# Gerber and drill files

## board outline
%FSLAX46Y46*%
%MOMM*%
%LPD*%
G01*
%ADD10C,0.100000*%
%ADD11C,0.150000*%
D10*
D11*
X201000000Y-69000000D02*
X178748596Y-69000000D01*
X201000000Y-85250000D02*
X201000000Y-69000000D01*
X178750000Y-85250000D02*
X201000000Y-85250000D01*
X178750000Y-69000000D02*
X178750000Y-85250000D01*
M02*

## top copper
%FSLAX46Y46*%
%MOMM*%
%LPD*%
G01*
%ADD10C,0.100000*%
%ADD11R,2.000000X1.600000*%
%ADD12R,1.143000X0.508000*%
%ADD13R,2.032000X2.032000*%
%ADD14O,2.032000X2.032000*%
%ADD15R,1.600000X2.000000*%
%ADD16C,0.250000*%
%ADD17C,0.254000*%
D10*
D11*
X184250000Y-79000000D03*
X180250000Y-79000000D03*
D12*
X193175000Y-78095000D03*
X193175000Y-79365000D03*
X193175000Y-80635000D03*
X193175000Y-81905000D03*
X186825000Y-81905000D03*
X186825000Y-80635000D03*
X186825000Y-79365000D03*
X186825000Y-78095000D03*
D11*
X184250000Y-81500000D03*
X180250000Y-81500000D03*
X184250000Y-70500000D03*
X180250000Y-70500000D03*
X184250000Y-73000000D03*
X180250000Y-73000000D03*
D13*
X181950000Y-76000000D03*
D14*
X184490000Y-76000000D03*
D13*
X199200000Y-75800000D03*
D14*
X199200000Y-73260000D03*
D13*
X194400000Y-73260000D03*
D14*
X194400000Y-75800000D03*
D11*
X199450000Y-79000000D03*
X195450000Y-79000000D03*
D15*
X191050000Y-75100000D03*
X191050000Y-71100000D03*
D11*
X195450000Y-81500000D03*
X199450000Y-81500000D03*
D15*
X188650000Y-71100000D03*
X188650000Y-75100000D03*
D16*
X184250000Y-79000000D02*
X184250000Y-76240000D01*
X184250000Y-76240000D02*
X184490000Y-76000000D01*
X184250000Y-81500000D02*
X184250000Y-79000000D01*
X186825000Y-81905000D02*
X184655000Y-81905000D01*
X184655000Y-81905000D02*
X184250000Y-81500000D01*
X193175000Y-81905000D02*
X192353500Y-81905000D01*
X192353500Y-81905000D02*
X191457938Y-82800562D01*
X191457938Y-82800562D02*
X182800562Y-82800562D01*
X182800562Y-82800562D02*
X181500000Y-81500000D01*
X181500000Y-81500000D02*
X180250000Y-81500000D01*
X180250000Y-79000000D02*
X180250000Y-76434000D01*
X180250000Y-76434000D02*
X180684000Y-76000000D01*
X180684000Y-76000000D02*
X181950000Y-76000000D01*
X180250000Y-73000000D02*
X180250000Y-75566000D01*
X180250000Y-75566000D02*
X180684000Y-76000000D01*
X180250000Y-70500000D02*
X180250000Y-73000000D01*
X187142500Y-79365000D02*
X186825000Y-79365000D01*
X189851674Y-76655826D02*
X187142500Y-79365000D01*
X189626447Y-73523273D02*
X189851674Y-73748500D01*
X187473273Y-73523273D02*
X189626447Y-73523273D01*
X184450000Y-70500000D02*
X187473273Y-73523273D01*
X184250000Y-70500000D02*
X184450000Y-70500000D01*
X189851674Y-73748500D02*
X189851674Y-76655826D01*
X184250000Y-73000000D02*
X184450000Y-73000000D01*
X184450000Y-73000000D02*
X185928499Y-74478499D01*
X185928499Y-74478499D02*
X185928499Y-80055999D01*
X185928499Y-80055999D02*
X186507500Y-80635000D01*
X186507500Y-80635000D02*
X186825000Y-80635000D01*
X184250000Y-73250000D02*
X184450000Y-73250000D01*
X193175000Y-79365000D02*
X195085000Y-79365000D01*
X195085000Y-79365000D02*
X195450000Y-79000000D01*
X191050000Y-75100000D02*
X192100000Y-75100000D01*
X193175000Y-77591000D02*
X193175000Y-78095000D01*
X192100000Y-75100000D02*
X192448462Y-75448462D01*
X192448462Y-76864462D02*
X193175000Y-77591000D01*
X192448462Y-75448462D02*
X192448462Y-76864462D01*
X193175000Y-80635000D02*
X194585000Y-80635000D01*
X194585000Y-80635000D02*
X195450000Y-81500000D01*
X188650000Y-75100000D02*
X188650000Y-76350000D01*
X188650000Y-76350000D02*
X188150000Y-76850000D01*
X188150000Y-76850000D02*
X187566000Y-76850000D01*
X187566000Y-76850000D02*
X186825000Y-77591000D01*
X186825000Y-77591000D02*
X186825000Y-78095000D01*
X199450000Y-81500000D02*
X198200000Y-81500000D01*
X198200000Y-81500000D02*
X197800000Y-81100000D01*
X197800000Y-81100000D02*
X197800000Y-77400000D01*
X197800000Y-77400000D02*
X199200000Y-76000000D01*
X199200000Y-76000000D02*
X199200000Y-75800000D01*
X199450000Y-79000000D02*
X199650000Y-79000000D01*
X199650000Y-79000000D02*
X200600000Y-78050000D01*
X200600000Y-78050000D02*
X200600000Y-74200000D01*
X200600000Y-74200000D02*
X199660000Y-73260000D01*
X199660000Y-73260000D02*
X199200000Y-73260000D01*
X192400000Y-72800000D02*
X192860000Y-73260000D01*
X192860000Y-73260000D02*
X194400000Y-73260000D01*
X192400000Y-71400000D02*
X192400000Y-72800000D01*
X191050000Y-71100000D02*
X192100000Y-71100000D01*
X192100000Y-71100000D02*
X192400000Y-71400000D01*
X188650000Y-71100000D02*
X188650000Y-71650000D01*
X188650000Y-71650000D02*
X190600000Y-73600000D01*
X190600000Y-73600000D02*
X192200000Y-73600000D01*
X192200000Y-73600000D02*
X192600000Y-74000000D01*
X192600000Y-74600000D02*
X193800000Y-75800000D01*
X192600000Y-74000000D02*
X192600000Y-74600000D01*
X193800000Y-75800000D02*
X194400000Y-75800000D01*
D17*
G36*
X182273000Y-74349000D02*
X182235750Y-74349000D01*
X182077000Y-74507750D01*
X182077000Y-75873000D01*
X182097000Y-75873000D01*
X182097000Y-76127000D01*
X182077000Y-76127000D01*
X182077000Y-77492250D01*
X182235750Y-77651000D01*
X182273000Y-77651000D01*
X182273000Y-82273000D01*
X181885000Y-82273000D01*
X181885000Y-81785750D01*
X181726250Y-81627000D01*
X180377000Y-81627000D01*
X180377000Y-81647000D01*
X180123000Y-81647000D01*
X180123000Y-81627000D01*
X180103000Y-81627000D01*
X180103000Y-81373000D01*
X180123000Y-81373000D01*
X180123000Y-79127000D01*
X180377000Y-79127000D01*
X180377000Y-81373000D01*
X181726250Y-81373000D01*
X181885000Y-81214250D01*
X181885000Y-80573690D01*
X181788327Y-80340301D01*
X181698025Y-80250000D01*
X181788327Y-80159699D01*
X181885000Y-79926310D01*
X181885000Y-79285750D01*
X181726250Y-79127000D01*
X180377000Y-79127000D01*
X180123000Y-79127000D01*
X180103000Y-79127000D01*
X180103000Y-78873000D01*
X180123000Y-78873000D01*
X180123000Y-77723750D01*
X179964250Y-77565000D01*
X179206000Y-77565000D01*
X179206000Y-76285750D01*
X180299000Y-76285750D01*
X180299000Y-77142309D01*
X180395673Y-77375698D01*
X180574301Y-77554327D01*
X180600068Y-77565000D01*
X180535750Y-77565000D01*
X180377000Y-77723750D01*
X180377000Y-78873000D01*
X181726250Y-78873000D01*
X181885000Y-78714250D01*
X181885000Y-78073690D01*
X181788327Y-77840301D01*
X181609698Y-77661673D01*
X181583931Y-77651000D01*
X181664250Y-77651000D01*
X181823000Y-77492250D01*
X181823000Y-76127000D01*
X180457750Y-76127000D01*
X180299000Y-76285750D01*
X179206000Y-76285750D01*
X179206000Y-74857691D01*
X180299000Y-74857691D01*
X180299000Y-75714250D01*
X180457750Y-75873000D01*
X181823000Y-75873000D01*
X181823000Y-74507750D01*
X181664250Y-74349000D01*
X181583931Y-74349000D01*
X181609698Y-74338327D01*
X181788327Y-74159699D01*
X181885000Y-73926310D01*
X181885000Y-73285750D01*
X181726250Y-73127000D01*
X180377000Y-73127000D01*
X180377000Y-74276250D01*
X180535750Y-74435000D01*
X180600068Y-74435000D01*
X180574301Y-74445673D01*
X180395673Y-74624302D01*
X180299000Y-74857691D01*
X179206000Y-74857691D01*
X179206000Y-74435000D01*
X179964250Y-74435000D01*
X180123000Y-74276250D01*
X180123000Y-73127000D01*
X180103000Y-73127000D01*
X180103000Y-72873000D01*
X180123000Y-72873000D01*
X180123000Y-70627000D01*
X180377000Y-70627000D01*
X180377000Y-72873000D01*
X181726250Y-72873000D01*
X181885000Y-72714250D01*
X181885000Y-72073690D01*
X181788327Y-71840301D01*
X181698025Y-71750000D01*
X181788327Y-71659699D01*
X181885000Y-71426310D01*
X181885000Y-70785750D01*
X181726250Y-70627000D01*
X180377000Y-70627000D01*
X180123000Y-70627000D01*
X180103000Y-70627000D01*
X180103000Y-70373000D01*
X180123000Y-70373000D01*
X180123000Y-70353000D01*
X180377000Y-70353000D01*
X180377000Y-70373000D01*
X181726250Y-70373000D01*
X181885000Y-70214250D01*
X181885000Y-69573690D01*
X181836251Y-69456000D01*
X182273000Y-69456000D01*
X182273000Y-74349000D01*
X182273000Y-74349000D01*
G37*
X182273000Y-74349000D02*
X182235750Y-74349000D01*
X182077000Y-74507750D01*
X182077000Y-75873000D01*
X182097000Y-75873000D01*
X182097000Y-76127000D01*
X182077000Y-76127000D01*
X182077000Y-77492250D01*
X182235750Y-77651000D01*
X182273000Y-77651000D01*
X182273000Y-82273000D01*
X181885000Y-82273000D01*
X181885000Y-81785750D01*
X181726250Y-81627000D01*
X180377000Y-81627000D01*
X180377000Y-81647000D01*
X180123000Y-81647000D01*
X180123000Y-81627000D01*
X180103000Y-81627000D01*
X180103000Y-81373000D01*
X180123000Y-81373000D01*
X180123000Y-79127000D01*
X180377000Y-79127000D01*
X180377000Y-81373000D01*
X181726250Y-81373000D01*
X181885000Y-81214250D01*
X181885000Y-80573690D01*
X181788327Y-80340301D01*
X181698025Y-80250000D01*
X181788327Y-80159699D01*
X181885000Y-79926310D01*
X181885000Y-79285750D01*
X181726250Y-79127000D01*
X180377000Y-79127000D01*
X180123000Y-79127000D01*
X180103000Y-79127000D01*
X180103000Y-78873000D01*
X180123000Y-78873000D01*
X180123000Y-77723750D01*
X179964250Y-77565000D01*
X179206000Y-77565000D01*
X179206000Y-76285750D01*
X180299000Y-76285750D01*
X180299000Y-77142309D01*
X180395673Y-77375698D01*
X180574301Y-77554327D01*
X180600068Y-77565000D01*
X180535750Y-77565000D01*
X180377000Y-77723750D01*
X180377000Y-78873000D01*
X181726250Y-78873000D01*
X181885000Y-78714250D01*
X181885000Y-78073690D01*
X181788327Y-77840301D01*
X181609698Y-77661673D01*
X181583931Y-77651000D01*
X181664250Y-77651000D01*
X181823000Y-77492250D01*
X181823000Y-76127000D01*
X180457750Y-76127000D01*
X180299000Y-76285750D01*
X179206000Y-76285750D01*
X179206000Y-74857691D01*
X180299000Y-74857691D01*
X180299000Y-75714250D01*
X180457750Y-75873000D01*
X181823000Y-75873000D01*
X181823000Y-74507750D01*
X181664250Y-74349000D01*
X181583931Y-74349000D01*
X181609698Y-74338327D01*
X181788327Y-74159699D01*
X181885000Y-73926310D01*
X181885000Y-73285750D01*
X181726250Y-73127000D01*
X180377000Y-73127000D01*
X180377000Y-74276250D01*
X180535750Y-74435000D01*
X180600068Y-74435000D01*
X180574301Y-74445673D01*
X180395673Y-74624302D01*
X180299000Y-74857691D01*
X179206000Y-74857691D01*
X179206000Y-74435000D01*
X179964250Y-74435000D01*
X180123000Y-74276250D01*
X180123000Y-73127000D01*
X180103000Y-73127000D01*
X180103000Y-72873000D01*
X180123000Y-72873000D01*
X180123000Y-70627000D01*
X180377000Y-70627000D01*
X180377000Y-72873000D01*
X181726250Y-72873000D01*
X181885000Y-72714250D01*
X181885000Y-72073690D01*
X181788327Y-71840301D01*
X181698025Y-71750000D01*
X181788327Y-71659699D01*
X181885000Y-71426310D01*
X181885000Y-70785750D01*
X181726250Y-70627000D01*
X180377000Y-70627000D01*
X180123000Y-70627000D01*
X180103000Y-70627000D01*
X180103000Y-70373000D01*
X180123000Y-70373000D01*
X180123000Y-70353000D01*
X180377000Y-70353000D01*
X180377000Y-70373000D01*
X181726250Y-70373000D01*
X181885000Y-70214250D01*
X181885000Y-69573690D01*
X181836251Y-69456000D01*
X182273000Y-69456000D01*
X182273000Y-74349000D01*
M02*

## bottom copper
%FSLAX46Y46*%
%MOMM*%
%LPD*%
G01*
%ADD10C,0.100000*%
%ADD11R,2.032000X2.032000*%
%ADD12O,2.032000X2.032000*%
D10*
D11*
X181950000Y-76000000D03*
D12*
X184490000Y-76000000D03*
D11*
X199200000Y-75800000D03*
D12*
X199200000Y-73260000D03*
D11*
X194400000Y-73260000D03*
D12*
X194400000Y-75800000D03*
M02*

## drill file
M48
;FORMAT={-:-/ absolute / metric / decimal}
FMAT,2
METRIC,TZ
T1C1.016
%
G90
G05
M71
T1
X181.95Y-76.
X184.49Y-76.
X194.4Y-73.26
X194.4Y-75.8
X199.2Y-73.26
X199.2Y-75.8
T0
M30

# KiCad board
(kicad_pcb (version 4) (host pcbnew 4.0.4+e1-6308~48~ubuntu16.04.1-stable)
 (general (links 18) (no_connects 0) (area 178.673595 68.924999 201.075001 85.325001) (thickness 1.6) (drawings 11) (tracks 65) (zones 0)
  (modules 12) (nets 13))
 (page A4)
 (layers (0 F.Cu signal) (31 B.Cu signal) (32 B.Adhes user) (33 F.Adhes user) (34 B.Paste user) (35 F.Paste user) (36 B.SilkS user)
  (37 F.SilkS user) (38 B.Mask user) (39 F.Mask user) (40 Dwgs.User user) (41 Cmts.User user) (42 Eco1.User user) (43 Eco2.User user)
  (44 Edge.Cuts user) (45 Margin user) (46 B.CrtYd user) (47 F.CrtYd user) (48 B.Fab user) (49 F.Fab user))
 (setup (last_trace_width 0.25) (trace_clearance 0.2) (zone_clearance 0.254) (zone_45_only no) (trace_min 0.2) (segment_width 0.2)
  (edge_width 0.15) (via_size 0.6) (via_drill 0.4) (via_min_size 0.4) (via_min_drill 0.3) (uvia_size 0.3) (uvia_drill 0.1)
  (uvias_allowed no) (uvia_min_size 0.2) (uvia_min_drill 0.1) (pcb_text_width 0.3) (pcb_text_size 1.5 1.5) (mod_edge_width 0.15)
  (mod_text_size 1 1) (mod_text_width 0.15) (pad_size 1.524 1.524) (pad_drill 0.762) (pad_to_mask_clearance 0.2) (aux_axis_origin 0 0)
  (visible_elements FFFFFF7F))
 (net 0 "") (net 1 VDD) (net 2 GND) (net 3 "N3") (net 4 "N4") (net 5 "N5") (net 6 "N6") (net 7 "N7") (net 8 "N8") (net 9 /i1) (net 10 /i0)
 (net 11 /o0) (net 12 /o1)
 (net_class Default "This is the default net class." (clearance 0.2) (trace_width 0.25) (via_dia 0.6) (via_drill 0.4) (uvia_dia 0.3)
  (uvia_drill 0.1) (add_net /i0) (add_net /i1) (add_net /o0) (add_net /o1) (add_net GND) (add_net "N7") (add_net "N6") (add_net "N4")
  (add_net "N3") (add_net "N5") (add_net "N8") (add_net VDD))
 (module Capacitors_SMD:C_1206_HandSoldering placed (layer F.Cu) (at 182.25 79 180)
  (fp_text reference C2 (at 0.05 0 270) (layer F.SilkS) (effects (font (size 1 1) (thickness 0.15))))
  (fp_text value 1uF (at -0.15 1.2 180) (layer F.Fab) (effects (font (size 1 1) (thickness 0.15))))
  (pad 1 smd rect (at -2 0 180) (size 2 1.6) (layers F.Cu F.Paste F.Mask) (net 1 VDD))
  (pad 2 smd rect (at 2 0 180) (size 2 1.6) (layers F.Cu F.Paste F.Mask) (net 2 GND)))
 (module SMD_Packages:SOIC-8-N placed (layer F.Cu) (at 190 80 270)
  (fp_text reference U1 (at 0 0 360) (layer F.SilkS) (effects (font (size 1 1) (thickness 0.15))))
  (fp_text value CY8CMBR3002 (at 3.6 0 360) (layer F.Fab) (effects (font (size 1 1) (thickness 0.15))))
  (pad 8 smd rect (at -1.905 -3.175 270) (size 0.508 1.143) (layers F.Cu F.Paste F.Mask) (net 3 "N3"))
  (pad 7 smd rect (at -0.635 -3.175 270) (size 0.508 1.143) (layers F.Cu F.Paste F.Mask) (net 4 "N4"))
  (pad 6 smd rect (at 0.635 -3.175 270) (size 0.508 1.143) (layers F.Cu F.Paste F.Mask) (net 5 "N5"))
  (pad 5 smd rect (at 1.905 -3.175 270) (size 0.508 1.143) (layers F.Cu F.Paste F.Mask) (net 2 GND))
  (pad 4 smd rect (at 1.905 3.175 270) (size 0.508 1.143) (layers F.Cu F.Paste F.Mask) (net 1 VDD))
  (pad 3 smd rect (at 0.635 3.175 270) (size 0.508 1.143) (layers F.Cu F.Paste F.Mask) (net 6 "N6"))
  (pad 2 smd rect (at -0.635 3.175 270) (size 0.508 1.143) (layers F.Cu F.Paste F.Mask) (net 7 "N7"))
  (pad 1 smd rect (at -1.905 3.175 270) (size 0.508 1.143) (layers F.Cu F.Paste F.Mask) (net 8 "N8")))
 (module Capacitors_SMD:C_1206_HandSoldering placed (layer F.Cu) (at 182.25 81.5 180)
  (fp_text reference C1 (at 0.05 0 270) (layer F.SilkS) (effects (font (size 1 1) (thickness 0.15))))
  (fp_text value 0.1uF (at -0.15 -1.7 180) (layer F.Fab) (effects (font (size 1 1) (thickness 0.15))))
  (pad 1 smd rect (at -2 0 180) (size 2 1.6) (layers F.Cu F.Paste F.Mask) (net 1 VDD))
  (pad 2 smd rect (at 2 0 180) (size 2 1.6) (layers F.Cu F.Paste F.Mask) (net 2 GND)))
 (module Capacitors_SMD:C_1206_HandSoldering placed (layer F.Cu) (at 182.25 70.5 180)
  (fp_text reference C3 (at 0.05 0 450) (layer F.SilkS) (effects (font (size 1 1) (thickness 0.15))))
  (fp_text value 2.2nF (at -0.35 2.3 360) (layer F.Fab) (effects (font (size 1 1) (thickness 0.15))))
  (pad 1 smd rect (at -2 0 180) (size 2 1.6) (layers F.Cu F.Paste F.Mask) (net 7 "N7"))
  (pad 2 smd rect (at 2 0 180) (size 2 1.6) (layers F.Cu F.Paste F.Mask) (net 2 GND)))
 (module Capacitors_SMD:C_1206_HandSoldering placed (layer F.Cu) (at 182.25 73 180)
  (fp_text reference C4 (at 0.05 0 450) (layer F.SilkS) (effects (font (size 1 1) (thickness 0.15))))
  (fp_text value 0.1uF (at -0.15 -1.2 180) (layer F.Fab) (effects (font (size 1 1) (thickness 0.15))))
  (pad 1 smd rect (at -2 0 180) (size 2 1.6) (layers F.Cu F.Paste F.Mask) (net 6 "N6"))
  (pad 2 smd rect (at 2 0 180) (size 2 1.6) (layers F.Cu F.Paste F.Mask) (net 2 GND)))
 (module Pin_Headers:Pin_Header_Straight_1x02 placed (layer F.Cu) (at 181.95 76 90)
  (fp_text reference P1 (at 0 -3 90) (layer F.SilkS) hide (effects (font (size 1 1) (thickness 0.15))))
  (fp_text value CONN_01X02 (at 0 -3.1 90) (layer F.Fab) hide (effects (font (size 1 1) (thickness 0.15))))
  (pad 1 thru_hole rect (at 0 0 90) (size 2.032 2.032) (drill 1.016) (layers *.Cu *.Mask F.SilkS) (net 2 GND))
  (pad 2 thru_hole oval (at 0 2.54 90) (size 2.032 2.032) (drill 1.016) (layers *.Cu *.Mask F.SilkS) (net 1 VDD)))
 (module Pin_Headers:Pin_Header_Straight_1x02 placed (layer F.Cu) (at 199.2 75.8 180)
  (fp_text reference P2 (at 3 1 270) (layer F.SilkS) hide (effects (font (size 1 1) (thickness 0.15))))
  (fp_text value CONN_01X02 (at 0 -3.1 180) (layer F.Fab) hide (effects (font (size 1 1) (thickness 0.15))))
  (pad 1 thru_hole rect (at 0 0 180) (size 2.032 2.032) (drill 1.016) (layers *.Cu *.Mask F.SilkS) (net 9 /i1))
  (pad 2 thru_hole oval (at 0 2.54 180) (size 2.032 2.032) (drill 1.016) (layers *.Cu *.Mask F.SilkS) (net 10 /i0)))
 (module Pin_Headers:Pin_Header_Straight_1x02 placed (layer F.Cu) (at 194.4 73.26)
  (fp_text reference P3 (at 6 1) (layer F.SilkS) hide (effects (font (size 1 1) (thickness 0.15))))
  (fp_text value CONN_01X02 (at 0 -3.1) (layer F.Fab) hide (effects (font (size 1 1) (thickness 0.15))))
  (pad 1 thru_hole rect (at 0 0) (size 2.032 2.032) (drill 1.016) (layers *.Cu *.Mask F.SilkS) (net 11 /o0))
  (pad 2 thru_hole oval (at 0 2.54) (size 2.032 2.032) (drill 1.016) (layers *.Cu *.Mask F.SilkS) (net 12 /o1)))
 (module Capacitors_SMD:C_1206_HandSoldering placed (layer F.Cu) (at 197.45 79 180)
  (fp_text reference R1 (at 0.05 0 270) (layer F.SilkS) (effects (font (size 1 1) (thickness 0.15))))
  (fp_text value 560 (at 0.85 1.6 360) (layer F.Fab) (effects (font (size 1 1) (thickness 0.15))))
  (pad 1 smd rect (at -2 0 180) (size 2 1.6) (layers F.Cu F.Paste F.Mask) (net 10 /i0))
  (pad 2 smd rect (at 2 0 180) (size 2 1.6) (layers F.Cu F.Paste F.Mask) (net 4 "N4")))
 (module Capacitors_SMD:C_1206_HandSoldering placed (layer F.Cu) (at 191.05 73.1 90)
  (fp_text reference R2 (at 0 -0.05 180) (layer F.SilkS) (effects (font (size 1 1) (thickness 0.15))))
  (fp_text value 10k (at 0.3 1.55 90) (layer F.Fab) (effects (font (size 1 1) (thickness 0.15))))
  (pad 1 smd rect (at -2 0 90) (size 2 1.6) (layers F.Cu F.Paste F.Mask) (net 3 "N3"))
  (pad 2 smd rect (at 2 0 90) (size 2 1.6) (layers F.Cu F.Paste F.Mask) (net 11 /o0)))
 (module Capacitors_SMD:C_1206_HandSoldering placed (layer F.Cu) (at 197.45 81.5)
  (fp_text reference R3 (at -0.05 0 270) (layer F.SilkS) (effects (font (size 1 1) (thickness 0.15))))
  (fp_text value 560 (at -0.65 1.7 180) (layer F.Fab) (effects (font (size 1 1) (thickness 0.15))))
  (pad 1 smd rect (at -2 0) (size 2 1.6) (layers F.Cu F.Paste F.Mask) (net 5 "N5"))
  (pad 2 smd rect (at 2 0) (size 2 1.6) (layers F.Cu F.Paste F.Mask) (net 9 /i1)))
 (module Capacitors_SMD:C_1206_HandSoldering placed (layer F.Cu) (at 188.65 73.1 270)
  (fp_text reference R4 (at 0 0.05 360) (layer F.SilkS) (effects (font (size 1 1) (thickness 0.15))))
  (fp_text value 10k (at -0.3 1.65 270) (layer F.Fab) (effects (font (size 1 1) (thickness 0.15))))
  (pad 1 smd rect (at -2 0 270) (size 2 1.6) (layers F.Cu F.Paste F.Mask) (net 12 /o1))
  (pad 2 smd rect (at 2 0 270) (size 2 1.6) (layers F.Cu F.Paste F.Mask) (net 8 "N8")))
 (gr_line (start 201 69) (end 178.748596 69) (layer Edge.Cuts) (width 0.15))
 (gr_line (start 201 85.25) (end 201 69) (layer Edge.Cuts) (width 0.15))
 (gr_line (start 178.75 85.25) (end 201 85.25) (layer Edge.Cuts) (width 0.15))
 (gr_line (start 178.75 69) (end 178.75 85.25) (layer Edge.Cuts) (width 0.15))
 (segment (start 184.25 79) (end 184.25 76.24) (width 0.25) (layer F.Cu) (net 1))
 (segment (start 184.25 76.24) (end 184.49 76) (width 0.25) (layer F.Cu) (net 1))
 (segment (start 184.25 81.5) (end 184.25 79) (width 0.25) (layer F.Cu) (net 1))
 (segment (start 186.825 81.905) (end 184.655 81.905) (width 0.25) (layer F.Cu) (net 1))
 (segment (start 184.655 81.905) (end 184.25 81.5) (width 0.25) (layer F.Cu) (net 1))
 (segment (start 193.175 81.905) (end 192.3535 81.905) (width 0.25) (layer F.Cu) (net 2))
 (segment (start 192.3535 81.905) (end 191.457938 82.800562) (width 0.25) (layer F.Cu) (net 2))
 (segment (start 191.457938 82.800562) (end 182.800562 82.800562) (width 0.25) (layer F.Cu) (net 2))
 (segment (start 182.800562 82.800562) (end 181.5 81.5) (width 0.25) (layer F.Cu) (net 2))
 (segment (start 181.5 81.5) (end 180.25 81.5) (width 0.25) (layer F.Cu) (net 2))
 (segment (start 180.25 79) (end 180.25 76.434) (width 0.25) (layer F.Cu) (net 2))
 (segment (start 180.25 76.434) (end 180.684 76) (width 0.25) (layer F.Cu) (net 2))
 (segment (start 180.684 76) (end 181.95 76) (width 0.25) (layer F.Cu) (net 2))
 (segment (start 180.25 73) (end 180.25 75.566) (width 0.25) (layer F.Cu) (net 2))
 (segment (start 180.25 75.566) (end 180.684 76) (width 0.25) (layer F.Cu) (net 2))
 (segment (start 180.25 70.5) (end 180.25 73) (width 0.25) (layer F.Cu) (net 2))
 (segment (start 187.1425 79.365) (end 186.825 79.365) (width 0.25) (layer F.Cu) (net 7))
 (segment (start 189.851674 76.655826) (end 187.1425 79.365) (width 0.25) (layer F.Cu) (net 7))
 (segment (start 189.626447 73.523273) (end 189.851674 73.7485) (width 0.25) (layer F.Cu) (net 7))
 (segment (start 187.473273 73.523273) (end 189.626447 73.523273) (width 0.25) (layer F.Cu) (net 7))
 (segment (start 184.45 70.5) (end 187.473273 73.523273) (width 0.25) (layer F.Cu) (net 7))
 (segment (start 184.25 70.5) (end 184.45 70.5) (width 0.25) (layer F.Cu) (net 7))
 (segment (start 189.851674 73.7485) (end 189.851674 76.655826) (width 0.25) (layer F.Cu) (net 7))
 (segment (start 184.25 73) (end 184.45 73) (width 0.25) (layer F.Cu) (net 6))
 (segment (start 184.45 73) (end 185.928499 74.478499) (width 0.25) (layer F.Cu) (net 6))
 (segment (start 185.928499 74.478499) (end 185.928499 80.055999) (width 0.25) (layer F.Cu) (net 6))
 (segment (start 185.928499 80.055999) (end 186.5075 80.635) (width 0.25) (layer F.Cu) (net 6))
 (segment (start 186.5075 80.635) (end 186.825 80.635) (width 0.25) (layer F.Cu) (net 6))
 (segment (start 184.25 73.25) (end 184.45 73.25) (width 0.25) (layer F.Cu) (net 6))
 (segment (start 193.175 79.365) (end 195.085 79.365) (width 0.25) (layer F.Cu) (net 4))
 (segment (start 195.085 79.365) (end 195.45 79) (width 0.25) (layer F.Cu) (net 4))
 (segment (start 191.05 75.1) (end 192.1 75.1) (width 0.25) (layer F.Cu) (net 3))
 (segment (start 193.175 77.591) (end 193.175 78.095) (width 0.25) (layer F.Cu) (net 3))
 (segment (start 192.1 75.1) (end 192.448462 75.448462) (width 0.25) (layer F.Cu) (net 3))
 (segment (start 192.448462 76.864462) (end 193.175 77.591) (width 0.25) (layer F.Cu) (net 3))
 (segment (start 192.448462 75.448462) (end 192.448462 76.864462) (width 0.25) (layer F.Cu) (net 3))
 (segment (start 193.175 80.635) (end 194.585 80.635) (width 0.25) (layer F.Cu) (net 5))
 (segment (start 194.585 80.635) (end 195.45 81.5) (width 0.25) (layer F.Cu) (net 5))
 (segment (start 188.65 75.1) (end 188.65 76.35) (width 0.25) (layer F.Cu) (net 8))
 (segment (start 188.65 76.35) (end 188.15 76.85) (width 0.25) (layer F.Cu) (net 8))
 (segment (start 188.15 76.85) (end 187.566 76.85) (width 0.25) (layer F.Cu) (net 8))
 (segment (start 187.566 76.85) (end 186.825 77.591) (width 0.25) (layer F.Cu) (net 8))
 (segment (start 186.825 77.591) (end 186.825 78.095) (width 0.25) (layer F.Cu) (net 8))
 (segment (start 199.45 81.5) (end 198.2 81.5) (width 0.25) (layer F.Cu) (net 9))
 (segment (start 198.2 81.5) (end 197.8 81.1) (width 0.25) (layer F.Cu) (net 9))
 (segment (start 197.8 81.1) (end 197.8 77.4) (width 0.25) (layer F.Cu) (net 9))
 (segment (start 197.8 77.4) (end 199.2 76) (width 0.25) (layer F.Cu) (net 9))
 (segment (start 199.2 76) (end 199.2 75.8) (width 0.25) (layer F.Cu) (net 9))
 (segment (start 199.45 79) (end 199.65 79) (width 0.25) (layer F.Cu) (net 10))
 (segment (start 199.65 79) (end 200.6 78.05) (width 0.25) (layer F.Cu) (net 10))
 (segment (start 200.6 78.05) (end 200.6 74.2) (width 0.25) (layer F.Cu) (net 10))
 (segment (start 200.6 74.2) (end 199.66 73.26) (width 0.25) (layer F.Cu) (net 10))
 (segment (start 199.66 73.26) (end 199.2 73.26) (width 0.25) (layer F.Cu) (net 10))
 (segment (start 192.4 72.8) (end 192.86 73.26) (width 0.25) (layer F.Cu) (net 11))
 (segment (start 192.86 73.26) (end 194.4 73.26) (width 0.25) (layer F.Cu) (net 11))
 (segment (start 192.4 71.4) (end 192.4 72.8) (width 0.25) (layer F.Cu) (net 11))
 (segment (start 191.05 71.1) (end 192.1 71.1) (width 0.25) (layer F.Cu) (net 11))
 (segment (start 192.1 71.1) (end 192.4 71.4) (width 0.25) (layer F.Cu) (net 11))
 (segment (start 188.65 71.1) (end 188.65 71.65) (width 0.25) (layer F.Cu) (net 12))
 (segment (start 188.65 71.65) (end 190.6 73.6) (width 0.25) (layer F.Cu) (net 12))
 (segment (start 190.6 73.6) (end 192.2 73.6) (width 0.25) (layer F.Cu) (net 12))
 (segment (start 192.2 73.6) (end 192.6 74) (width 0.25) (layer F.Cu) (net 12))
 (segment (start 192.6 74.6) (end 193.8 75.8) (width 0.25) (layer F.Cu) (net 12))
 (segment (start 192.6 74) (end 192.6 74.6) (width 0.25) (layer F.Cu) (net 12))
 (segment (start 193.8 75.8) (end 194.4 75.8) (width 0.25) (layer F.Cu) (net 12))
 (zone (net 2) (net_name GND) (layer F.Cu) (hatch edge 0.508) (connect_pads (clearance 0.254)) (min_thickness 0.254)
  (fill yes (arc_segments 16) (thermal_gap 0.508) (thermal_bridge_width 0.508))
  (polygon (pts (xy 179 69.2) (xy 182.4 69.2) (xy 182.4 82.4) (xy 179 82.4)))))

